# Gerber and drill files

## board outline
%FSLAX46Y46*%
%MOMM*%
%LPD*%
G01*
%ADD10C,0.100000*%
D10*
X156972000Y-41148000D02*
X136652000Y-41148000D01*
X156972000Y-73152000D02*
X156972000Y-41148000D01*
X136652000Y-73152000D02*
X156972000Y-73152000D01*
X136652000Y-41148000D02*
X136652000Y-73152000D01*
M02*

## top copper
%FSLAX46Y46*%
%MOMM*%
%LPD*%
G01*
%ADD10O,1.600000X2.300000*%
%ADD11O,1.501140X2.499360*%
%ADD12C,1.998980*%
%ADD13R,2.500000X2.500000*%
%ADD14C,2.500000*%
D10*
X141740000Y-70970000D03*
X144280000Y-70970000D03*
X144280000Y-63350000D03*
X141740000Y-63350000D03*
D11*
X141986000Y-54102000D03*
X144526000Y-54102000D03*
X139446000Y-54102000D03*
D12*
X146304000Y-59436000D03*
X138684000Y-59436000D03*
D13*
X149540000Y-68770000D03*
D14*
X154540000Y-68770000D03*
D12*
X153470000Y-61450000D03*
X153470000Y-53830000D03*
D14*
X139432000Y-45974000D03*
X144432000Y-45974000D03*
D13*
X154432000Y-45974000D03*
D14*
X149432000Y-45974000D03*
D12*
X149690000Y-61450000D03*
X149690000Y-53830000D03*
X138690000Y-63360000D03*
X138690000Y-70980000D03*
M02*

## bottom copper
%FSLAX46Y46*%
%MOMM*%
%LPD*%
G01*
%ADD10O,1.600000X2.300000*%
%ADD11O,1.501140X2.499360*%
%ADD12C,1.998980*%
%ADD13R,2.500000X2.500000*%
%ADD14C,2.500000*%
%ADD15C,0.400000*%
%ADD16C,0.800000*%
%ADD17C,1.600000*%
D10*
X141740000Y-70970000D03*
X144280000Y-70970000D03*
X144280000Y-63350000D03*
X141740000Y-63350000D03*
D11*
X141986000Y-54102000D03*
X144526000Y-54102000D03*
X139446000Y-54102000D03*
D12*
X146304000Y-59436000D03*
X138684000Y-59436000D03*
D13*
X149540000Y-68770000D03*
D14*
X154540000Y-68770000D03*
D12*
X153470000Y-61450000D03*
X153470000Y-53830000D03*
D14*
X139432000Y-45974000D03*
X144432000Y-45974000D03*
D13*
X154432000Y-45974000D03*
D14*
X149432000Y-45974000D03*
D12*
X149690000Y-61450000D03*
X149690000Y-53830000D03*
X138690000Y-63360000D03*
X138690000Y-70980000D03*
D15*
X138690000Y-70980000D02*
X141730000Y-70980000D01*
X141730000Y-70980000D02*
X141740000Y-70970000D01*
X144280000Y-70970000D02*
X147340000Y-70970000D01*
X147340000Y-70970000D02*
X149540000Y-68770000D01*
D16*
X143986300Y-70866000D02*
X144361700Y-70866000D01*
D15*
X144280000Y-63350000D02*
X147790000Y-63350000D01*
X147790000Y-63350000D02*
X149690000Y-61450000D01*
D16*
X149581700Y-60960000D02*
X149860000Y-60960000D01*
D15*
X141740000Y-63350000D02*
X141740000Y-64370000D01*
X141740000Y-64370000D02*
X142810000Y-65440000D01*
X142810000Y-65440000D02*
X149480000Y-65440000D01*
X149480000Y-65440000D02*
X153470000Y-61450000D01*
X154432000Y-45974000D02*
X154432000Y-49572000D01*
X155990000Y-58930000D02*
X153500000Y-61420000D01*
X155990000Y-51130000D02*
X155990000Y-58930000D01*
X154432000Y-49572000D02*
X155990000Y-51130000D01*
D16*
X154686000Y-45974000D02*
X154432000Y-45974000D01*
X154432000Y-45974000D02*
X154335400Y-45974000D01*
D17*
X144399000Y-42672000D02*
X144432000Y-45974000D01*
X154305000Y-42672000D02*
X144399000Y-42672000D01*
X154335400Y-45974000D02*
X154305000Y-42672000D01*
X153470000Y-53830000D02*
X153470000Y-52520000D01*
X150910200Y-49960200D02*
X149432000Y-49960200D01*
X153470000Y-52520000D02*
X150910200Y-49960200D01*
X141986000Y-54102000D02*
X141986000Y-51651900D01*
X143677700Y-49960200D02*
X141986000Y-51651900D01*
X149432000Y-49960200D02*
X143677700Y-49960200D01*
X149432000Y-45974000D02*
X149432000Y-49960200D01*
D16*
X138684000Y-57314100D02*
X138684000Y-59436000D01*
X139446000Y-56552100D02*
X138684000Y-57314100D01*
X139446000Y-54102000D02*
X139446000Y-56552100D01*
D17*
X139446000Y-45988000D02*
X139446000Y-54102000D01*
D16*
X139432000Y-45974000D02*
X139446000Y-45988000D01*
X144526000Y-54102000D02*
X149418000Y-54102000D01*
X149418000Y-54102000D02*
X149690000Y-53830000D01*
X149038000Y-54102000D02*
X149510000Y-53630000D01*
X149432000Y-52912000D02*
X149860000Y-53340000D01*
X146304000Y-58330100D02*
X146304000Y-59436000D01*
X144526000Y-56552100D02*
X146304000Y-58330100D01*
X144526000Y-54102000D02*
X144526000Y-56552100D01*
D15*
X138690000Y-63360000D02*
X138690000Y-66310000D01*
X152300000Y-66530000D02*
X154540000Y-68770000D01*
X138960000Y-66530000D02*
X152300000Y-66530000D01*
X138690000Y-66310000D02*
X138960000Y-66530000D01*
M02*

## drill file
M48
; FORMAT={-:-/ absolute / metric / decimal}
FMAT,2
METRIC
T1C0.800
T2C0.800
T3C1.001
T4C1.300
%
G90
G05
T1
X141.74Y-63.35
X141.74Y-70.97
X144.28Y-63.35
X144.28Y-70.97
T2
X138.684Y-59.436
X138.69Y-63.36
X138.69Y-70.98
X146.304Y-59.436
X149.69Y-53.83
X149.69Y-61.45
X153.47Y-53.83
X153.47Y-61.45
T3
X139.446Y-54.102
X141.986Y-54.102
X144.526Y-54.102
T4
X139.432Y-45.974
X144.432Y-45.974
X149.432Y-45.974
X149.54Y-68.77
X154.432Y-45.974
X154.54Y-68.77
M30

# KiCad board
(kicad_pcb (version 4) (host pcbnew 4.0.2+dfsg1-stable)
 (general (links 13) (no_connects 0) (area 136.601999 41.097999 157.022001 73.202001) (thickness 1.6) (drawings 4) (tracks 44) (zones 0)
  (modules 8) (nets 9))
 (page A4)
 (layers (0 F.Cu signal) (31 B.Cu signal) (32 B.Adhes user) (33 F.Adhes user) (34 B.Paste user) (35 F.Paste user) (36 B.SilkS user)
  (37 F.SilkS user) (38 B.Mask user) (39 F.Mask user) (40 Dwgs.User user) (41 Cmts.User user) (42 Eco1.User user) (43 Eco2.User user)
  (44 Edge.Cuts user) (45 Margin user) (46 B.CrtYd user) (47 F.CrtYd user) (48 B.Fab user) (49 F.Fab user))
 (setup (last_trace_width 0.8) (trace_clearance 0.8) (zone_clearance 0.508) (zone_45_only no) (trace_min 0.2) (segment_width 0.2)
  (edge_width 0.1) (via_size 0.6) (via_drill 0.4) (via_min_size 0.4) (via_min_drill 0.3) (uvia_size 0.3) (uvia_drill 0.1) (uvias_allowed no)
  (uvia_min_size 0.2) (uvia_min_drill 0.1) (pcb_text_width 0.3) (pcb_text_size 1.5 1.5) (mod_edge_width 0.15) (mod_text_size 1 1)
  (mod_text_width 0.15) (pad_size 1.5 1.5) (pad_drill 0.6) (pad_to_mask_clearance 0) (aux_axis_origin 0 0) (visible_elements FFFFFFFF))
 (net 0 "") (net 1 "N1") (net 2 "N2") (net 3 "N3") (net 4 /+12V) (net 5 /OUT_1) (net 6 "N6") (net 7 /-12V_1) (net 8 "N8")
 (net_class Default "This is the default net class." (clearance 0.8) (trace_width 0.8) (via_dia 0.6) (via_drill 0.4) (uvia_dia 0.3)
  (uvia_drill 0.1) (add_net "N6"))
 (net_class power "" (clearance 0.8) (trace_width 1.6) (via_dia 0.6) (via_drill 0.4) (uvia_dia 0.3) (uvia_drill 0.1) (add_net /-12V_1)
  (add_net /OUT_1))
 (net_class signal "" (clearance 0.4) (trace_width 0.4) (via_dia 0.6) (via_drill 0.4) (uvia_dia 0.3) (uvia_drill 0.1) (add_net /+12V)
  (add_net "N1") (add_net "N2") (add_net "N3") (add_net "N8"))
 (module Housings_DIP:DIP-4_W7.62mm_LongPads (layer F.Cu) (at 141.74 70.97 90)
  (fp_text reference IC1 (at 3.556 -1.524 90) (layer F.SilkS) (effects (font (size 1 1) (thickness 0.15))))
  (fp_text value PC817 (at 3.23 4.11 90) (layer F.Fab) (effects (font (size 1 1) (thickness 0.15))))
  (pad 1 thru_hole oval (at 0 0 90) (size 2.3 1.6) (drill 0.8) (layers *.Cu *.Mask F.SilkS) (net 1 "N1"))
  (pad 2 thru_hole oval (at 0 2.54 90) (size 2.3 1.6) (drill 0.8) (layers *.Cu *.Mask F.SilkS) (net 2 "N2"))
  (pad 3 thru_hole oval (at 7.62 2.54 90) (size 2.3 1.6) (drill 0.8) (layers *.Cu *.Mask F.SilkS) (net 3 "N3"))
  (pad 4 thru_hole oval (at 7.62 0 90) (size 2.3 1.6) (drill 0.8) (layers *.Cu *.Mask F.SilkS) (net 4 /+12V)))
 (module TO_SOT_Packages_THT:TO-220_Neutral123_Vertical (layer F.Cu) (at 141.986 54.102 180)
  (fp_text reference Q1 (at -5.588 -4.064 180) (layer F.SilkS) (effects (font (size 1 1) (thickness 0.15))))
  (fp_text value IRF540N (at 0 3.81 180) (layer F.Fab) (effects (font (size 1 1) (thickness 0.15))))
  (pad 2 thru_hole oval (at 0 0 270) (size 2.49936 1.50114) (drill 1.00076) (layers *.Cu *.Mask F.SilkS) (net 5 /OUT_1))
  (pad 1 thru_hole oval (at -2.54 0 270) (size 2.49936 1.50114) (drill 1.00076) (layers *.Cu *.Mask F.SilkS) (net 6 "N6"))
  (pad 3 thru_hole oval (at 2.54 0 270) (size 2.49936 1.50114) (drill 1.00076) (layers *.Cu *.Mask F.SilkS) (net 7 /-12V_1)))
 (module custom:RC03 (layer F.Cu) (at 142.494 59.436 180) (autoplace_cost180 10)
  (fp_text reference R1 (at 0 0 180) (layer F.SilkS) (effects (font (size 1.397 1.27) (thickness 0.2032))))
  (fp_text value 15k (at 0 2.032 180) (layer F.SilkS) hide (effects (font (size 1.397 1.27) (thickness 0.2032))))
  (pad 1 thru_hole circle (at -3.81 0 180) (size 1.99898 1.99898) (drill 0.8001) (layers *.Cu *.Mask F.SilkS) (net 6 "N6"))
  (pad 2 thru_hole circle (at 3.81 0 180) (size 1.99898 1.99898) (drill 0.8001) (layers *.Cu *.Mask F.SilkS) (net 7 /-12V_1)))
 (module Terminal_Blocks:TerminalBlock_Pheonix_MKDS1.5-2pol (layer F.Cu) (at 149.54 68.77)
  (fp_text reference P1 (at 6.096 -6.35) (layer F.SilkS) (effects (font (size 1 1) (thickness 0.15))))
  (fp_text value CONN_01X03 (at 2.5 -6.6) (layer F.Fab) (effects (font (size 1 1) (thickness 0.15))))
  (pad 1 thru_hole rect (at 0 0) (size 2.5 2.5) (drill 1.3) (layers *.Cu *.Mask F.SilkS) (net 2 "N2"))
  (pad 2 thru_hole circle (at 5 0) (size 2.5 2.5) (drill 1.3) (layers *.Cu *.Mask F.SilkS) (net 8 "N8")))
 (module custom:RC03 (layer F.Cu) (at 153.47 57.64 90) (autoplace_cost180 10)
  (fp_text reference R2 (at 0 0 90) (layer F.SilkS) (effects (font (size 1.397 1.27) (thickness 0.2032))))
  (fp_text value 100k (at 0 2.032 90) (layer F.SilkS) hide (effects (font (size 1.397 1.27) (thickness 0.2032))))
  (pad 1 thru_hole circle (at -3.81 0 90) (size 1.99898 1.99898) (drill 0.8001) (layers *.Cu *.Mask F.SilkS) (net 4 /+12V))
  (pad 2 thru_hole circle (at 3.81 0 90) (size 1.99898 1.99898) (drill 0.8001) (layers *.Cu *.Mask F.SilkS) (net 5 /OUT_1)))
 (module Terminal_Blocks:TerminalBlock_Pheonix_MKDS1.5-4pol (layer F.Cu) (at 154.432 45.974 180)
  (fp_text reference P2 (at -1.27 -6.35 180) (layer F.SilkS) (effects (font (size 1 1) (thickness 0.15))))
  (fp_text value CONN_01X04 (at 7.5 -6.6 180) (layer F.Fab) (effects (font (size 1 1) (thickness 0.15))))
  (pad 4 thru_hole circle (at 15 0 180) (size 2.5 2.5) (drill 1.3) (layers *.Cu *.Mask F.SilkS) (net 7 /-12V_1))
  (pad 3 thru_hole circle (at 10 0 180) (size 2.5 2.5) (drill 1.3) (layers *.Cu *.Mask F.SilkS) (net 4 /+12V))
  (pad 1 thru_hole rect (at 0 0 180) (size 2.5 2.5) (drill 1.3) (layers *.Cu *.Mask F.SilkS) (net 4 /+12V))
  (pad 2 thru_hole circle (at 5 0 180) (size 2.5 2.5) (drill 1.3) (layers *.Cu *.Mask F.SilkS) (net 5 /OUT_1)))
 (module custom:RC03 (layer F.Cu) (at 149.69 57.64 90) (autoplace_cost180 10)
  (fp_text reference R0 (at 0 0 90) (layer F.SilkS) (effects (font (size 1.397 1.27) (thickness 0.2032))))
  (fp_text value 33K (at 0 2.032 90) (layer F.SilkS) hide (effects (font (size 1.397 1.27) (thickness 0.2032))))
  (pad 1 thru_hole circle (at -3.81 0 90) (size 1.99898 1.99898) (drill 0.8001) (layers *.Cu *.Mask F.SilkS) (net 3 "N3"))
  (pad 2 thru_hole circle (at 3.81 0 90) (size 1.99898 1.99898) (drill 0.8001) (layers *.Cu *.Mask F.SilkS) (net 6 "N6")))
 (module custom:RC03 (layer F.Cu) (at 138.69 67.17 270) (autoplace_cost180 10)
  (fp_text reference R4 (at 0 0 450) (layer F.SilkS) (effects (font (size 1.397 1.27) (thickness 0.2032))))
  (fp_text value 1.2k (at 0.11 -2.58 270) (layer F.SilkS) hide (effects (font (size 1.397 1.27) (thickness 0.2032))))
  (pad 1 thru_hole circle (at -3.81 0 270) (size 1.99898 1.99898) (drill 0.8001) (layers *.Cu *.Mask F.SilkS) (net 8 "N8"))
  (pad 2 thru_hole circle (at 3.81 0 270) (size 1.99898 1.99898) (drill 0.8001) (layers *.Cu *.Mask F.SilkS) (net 1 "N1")))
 (gr_line (start 156.972 41.148) (end 136.652 41.148) (angle 90) (layer Edge.Cuts) (width 0.1))
 (gr_line (start 156.972 73.152) (end 156.972 41.148) (angle 90) (layer Edge.Cuts) (width 0.1))
 (gr_line (start 136.652 73.152) (end 156.972 73.152) (angle 90) (layer Edge.Cuts) (width 0.1))
 (gr_line (start 136.652 41.148) (end 136.652 73.152) (angle 90) (layer Edge.Cuts) (width 0.1))
 (segment (start 138.69 70.98) (end 141.73 70.98) (width 0.4) (layer B.Cu) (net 1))
 (segment (start 141.73 70.98) (end 141.74 70.97) (width 0.4) (layer B.Cu) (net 1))
 (segment (start 144.28 70.97) (end 147.34 70.97) (width 0.4) (layer B.Cu) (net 2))
 (segment (start 147.34 70.97) (end 149.54 68.77) (width 0.4) (layer B.Cu) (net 2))
 (segment (start 143.9863 70.866) (end 144.3617 70.866) (width 0.8) (layer B.Cu) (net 2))
 (segment (start 144.28 63.35) (end 147.79 63.35) (width 0.4) (layer B.Cu) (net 3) (status 400000))
 (segment (start 147.79 63.35) (end 149.69 61.45) (width 0.4) (layer B.Cu) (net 3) (status 800000))
 (segment (start 149.5817 60.96) (end 149.86 60.96) (width 0.8) (layer B.Cu) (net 3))
 (segment (start 141.74 63.35) (end 141.74 64.37) (width 0.4) (layer B.Cu) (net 4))
 (segment (start 141.74 64.37) (end 142.81 65.44) (width 0.4) (layer B.Cu) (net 4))
 (segment (start 142.81 65.44) (end 149.48 65.44) (width 0.4) (layer B.Cu) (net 4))
 (segment (start 149.48 65.44) (end 153.47 61.45) (width 0.4) (layer B.Cu) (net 4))
 (segment (start 154.432 45.974) (end 154.432 49.572) (width 0.4) (layer B.Cu) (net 4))
 (segment (start 155.99 58.93) (end 153.5 61.42) (width 0.4) (layer B.Cu) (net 4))
 (segment (start 155.99 51.13) (end 155.99 58.93) (width 0.4) (layer B.Cu) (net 4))
 (segment (start 154.432 49.572) (end 155.99 51.13) (width 0.4) (layer B.Cu) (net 4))
 (segment (start 154.686 45.974) (end 154.432 45.974) (width 0.8) (layer B.Cu) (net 4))
 (segment (start 154.432 45.974) (end 154.3354 45.974) (width 0.8) (layer B.Cu) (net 4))
 (segment (start 144.399 42.672) (end 144.432 45.974) (width 1.6) (layer B.Cu) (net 4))
 (segment (start 154.305 42.672) (end 144.399 42.672) (width 1.6) (layer B.Cu) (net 4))
 (segment (start 154.3354 45.974) (end 154.305 42.672) (width 1.6) (layer B.Cu) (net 4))
 (segment (start 153.47 53.83) (end 153.47 52.52) (width 1.6) (layer B.Cu) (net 5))
 (segment (start 150.9102 49.9602) (end 149.432 49.9602) (width 1.6) (layer B.Cu) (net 5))
 (segment (start 153.47 52.52) (end 150.9102 49.9602) (width 1.6) (layer B.Cu) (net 5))
 (segment (start 141.986 54.102) (end 141.986 51.6519) (width 1.6) (layer B.Cu) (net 5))
 (segment (start 143.6777 49.9602) (end 141.986 51.6519) (width 1.6) (layer B.Cu) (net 5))
 (segment (start 149.432 49.9602) (end 143.6777 49.9602) (width 1.6) (layer B.Cu) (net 5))
 (segment (start 149.432 45.974) (end 149.432 49.9602) (width 1.6) (layer B.Cu) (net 5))
 (segment (start 138.684 57.3141) (end 138.684 59.436) (width 0.8) (layer B.Cu) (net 7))
 (segment (start 139.446 56.5521) (end 138.684 57.3141) (width 0.8) (layer B.Cu) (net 7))
 (segment (start 139.446 54.102) (end 139.446 56.5521) (width 0.8) (layer B.Cu) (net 7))
 (segment (start 139.446 45.988) (end 139.446 54.102) (width 1.6) (layer B.Cu) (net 7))
 (segment (start 139.432 45.974) (end 139.446 45.988) (width 0.8) (layer B.Cu) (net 7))
 (segment (start 144.526 54.102) (end 149.418 54.102) (width 0.8) (layer B.Cu) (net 6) (status C00000))
 (segment (start 149.418 54.102) (end 149.69 53.83) (width 0.8) (layer B.Cu) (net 6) (status C00000))
 (segment (start 149.038 54.102) (end 149.51 53.63) (width 0.8) (layer B.Cu) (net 6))
 (segment (start 149.432 52.912) (end 149.86 53.34) (width 0.8) (layer B.Cu) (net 6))
 (segment (start 146.304 58.3301) (end 146.304 59.436) (width 0.8) (layer B.Cu) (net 6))
 (segment (start 144.526 56.5521) (end 146.304 58.3301) (width 0.8) (layer B.Cu) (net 6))
 (segment (start 144.526 54.102) (end 144.526 56.5521) (width 0.8) (layer B.Cu) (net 6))
 (segment (start 138.69 63.36) (end 138.69 66.31) (width 0.4) (layer B.Cu) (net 8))
 (segment (start 152.3 66.53) (end 154.54 68.77) (width 0.4) (layer B.Cu) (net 8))
 (segment (start 138.96 66.53) (end 152.3 66.53) (width 0.4) (layer B.Cu) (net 8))
 (segment (start 138.69 66.31) (end 138.96 66.53) (width 0.4) (layer B.Cu) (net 8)))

